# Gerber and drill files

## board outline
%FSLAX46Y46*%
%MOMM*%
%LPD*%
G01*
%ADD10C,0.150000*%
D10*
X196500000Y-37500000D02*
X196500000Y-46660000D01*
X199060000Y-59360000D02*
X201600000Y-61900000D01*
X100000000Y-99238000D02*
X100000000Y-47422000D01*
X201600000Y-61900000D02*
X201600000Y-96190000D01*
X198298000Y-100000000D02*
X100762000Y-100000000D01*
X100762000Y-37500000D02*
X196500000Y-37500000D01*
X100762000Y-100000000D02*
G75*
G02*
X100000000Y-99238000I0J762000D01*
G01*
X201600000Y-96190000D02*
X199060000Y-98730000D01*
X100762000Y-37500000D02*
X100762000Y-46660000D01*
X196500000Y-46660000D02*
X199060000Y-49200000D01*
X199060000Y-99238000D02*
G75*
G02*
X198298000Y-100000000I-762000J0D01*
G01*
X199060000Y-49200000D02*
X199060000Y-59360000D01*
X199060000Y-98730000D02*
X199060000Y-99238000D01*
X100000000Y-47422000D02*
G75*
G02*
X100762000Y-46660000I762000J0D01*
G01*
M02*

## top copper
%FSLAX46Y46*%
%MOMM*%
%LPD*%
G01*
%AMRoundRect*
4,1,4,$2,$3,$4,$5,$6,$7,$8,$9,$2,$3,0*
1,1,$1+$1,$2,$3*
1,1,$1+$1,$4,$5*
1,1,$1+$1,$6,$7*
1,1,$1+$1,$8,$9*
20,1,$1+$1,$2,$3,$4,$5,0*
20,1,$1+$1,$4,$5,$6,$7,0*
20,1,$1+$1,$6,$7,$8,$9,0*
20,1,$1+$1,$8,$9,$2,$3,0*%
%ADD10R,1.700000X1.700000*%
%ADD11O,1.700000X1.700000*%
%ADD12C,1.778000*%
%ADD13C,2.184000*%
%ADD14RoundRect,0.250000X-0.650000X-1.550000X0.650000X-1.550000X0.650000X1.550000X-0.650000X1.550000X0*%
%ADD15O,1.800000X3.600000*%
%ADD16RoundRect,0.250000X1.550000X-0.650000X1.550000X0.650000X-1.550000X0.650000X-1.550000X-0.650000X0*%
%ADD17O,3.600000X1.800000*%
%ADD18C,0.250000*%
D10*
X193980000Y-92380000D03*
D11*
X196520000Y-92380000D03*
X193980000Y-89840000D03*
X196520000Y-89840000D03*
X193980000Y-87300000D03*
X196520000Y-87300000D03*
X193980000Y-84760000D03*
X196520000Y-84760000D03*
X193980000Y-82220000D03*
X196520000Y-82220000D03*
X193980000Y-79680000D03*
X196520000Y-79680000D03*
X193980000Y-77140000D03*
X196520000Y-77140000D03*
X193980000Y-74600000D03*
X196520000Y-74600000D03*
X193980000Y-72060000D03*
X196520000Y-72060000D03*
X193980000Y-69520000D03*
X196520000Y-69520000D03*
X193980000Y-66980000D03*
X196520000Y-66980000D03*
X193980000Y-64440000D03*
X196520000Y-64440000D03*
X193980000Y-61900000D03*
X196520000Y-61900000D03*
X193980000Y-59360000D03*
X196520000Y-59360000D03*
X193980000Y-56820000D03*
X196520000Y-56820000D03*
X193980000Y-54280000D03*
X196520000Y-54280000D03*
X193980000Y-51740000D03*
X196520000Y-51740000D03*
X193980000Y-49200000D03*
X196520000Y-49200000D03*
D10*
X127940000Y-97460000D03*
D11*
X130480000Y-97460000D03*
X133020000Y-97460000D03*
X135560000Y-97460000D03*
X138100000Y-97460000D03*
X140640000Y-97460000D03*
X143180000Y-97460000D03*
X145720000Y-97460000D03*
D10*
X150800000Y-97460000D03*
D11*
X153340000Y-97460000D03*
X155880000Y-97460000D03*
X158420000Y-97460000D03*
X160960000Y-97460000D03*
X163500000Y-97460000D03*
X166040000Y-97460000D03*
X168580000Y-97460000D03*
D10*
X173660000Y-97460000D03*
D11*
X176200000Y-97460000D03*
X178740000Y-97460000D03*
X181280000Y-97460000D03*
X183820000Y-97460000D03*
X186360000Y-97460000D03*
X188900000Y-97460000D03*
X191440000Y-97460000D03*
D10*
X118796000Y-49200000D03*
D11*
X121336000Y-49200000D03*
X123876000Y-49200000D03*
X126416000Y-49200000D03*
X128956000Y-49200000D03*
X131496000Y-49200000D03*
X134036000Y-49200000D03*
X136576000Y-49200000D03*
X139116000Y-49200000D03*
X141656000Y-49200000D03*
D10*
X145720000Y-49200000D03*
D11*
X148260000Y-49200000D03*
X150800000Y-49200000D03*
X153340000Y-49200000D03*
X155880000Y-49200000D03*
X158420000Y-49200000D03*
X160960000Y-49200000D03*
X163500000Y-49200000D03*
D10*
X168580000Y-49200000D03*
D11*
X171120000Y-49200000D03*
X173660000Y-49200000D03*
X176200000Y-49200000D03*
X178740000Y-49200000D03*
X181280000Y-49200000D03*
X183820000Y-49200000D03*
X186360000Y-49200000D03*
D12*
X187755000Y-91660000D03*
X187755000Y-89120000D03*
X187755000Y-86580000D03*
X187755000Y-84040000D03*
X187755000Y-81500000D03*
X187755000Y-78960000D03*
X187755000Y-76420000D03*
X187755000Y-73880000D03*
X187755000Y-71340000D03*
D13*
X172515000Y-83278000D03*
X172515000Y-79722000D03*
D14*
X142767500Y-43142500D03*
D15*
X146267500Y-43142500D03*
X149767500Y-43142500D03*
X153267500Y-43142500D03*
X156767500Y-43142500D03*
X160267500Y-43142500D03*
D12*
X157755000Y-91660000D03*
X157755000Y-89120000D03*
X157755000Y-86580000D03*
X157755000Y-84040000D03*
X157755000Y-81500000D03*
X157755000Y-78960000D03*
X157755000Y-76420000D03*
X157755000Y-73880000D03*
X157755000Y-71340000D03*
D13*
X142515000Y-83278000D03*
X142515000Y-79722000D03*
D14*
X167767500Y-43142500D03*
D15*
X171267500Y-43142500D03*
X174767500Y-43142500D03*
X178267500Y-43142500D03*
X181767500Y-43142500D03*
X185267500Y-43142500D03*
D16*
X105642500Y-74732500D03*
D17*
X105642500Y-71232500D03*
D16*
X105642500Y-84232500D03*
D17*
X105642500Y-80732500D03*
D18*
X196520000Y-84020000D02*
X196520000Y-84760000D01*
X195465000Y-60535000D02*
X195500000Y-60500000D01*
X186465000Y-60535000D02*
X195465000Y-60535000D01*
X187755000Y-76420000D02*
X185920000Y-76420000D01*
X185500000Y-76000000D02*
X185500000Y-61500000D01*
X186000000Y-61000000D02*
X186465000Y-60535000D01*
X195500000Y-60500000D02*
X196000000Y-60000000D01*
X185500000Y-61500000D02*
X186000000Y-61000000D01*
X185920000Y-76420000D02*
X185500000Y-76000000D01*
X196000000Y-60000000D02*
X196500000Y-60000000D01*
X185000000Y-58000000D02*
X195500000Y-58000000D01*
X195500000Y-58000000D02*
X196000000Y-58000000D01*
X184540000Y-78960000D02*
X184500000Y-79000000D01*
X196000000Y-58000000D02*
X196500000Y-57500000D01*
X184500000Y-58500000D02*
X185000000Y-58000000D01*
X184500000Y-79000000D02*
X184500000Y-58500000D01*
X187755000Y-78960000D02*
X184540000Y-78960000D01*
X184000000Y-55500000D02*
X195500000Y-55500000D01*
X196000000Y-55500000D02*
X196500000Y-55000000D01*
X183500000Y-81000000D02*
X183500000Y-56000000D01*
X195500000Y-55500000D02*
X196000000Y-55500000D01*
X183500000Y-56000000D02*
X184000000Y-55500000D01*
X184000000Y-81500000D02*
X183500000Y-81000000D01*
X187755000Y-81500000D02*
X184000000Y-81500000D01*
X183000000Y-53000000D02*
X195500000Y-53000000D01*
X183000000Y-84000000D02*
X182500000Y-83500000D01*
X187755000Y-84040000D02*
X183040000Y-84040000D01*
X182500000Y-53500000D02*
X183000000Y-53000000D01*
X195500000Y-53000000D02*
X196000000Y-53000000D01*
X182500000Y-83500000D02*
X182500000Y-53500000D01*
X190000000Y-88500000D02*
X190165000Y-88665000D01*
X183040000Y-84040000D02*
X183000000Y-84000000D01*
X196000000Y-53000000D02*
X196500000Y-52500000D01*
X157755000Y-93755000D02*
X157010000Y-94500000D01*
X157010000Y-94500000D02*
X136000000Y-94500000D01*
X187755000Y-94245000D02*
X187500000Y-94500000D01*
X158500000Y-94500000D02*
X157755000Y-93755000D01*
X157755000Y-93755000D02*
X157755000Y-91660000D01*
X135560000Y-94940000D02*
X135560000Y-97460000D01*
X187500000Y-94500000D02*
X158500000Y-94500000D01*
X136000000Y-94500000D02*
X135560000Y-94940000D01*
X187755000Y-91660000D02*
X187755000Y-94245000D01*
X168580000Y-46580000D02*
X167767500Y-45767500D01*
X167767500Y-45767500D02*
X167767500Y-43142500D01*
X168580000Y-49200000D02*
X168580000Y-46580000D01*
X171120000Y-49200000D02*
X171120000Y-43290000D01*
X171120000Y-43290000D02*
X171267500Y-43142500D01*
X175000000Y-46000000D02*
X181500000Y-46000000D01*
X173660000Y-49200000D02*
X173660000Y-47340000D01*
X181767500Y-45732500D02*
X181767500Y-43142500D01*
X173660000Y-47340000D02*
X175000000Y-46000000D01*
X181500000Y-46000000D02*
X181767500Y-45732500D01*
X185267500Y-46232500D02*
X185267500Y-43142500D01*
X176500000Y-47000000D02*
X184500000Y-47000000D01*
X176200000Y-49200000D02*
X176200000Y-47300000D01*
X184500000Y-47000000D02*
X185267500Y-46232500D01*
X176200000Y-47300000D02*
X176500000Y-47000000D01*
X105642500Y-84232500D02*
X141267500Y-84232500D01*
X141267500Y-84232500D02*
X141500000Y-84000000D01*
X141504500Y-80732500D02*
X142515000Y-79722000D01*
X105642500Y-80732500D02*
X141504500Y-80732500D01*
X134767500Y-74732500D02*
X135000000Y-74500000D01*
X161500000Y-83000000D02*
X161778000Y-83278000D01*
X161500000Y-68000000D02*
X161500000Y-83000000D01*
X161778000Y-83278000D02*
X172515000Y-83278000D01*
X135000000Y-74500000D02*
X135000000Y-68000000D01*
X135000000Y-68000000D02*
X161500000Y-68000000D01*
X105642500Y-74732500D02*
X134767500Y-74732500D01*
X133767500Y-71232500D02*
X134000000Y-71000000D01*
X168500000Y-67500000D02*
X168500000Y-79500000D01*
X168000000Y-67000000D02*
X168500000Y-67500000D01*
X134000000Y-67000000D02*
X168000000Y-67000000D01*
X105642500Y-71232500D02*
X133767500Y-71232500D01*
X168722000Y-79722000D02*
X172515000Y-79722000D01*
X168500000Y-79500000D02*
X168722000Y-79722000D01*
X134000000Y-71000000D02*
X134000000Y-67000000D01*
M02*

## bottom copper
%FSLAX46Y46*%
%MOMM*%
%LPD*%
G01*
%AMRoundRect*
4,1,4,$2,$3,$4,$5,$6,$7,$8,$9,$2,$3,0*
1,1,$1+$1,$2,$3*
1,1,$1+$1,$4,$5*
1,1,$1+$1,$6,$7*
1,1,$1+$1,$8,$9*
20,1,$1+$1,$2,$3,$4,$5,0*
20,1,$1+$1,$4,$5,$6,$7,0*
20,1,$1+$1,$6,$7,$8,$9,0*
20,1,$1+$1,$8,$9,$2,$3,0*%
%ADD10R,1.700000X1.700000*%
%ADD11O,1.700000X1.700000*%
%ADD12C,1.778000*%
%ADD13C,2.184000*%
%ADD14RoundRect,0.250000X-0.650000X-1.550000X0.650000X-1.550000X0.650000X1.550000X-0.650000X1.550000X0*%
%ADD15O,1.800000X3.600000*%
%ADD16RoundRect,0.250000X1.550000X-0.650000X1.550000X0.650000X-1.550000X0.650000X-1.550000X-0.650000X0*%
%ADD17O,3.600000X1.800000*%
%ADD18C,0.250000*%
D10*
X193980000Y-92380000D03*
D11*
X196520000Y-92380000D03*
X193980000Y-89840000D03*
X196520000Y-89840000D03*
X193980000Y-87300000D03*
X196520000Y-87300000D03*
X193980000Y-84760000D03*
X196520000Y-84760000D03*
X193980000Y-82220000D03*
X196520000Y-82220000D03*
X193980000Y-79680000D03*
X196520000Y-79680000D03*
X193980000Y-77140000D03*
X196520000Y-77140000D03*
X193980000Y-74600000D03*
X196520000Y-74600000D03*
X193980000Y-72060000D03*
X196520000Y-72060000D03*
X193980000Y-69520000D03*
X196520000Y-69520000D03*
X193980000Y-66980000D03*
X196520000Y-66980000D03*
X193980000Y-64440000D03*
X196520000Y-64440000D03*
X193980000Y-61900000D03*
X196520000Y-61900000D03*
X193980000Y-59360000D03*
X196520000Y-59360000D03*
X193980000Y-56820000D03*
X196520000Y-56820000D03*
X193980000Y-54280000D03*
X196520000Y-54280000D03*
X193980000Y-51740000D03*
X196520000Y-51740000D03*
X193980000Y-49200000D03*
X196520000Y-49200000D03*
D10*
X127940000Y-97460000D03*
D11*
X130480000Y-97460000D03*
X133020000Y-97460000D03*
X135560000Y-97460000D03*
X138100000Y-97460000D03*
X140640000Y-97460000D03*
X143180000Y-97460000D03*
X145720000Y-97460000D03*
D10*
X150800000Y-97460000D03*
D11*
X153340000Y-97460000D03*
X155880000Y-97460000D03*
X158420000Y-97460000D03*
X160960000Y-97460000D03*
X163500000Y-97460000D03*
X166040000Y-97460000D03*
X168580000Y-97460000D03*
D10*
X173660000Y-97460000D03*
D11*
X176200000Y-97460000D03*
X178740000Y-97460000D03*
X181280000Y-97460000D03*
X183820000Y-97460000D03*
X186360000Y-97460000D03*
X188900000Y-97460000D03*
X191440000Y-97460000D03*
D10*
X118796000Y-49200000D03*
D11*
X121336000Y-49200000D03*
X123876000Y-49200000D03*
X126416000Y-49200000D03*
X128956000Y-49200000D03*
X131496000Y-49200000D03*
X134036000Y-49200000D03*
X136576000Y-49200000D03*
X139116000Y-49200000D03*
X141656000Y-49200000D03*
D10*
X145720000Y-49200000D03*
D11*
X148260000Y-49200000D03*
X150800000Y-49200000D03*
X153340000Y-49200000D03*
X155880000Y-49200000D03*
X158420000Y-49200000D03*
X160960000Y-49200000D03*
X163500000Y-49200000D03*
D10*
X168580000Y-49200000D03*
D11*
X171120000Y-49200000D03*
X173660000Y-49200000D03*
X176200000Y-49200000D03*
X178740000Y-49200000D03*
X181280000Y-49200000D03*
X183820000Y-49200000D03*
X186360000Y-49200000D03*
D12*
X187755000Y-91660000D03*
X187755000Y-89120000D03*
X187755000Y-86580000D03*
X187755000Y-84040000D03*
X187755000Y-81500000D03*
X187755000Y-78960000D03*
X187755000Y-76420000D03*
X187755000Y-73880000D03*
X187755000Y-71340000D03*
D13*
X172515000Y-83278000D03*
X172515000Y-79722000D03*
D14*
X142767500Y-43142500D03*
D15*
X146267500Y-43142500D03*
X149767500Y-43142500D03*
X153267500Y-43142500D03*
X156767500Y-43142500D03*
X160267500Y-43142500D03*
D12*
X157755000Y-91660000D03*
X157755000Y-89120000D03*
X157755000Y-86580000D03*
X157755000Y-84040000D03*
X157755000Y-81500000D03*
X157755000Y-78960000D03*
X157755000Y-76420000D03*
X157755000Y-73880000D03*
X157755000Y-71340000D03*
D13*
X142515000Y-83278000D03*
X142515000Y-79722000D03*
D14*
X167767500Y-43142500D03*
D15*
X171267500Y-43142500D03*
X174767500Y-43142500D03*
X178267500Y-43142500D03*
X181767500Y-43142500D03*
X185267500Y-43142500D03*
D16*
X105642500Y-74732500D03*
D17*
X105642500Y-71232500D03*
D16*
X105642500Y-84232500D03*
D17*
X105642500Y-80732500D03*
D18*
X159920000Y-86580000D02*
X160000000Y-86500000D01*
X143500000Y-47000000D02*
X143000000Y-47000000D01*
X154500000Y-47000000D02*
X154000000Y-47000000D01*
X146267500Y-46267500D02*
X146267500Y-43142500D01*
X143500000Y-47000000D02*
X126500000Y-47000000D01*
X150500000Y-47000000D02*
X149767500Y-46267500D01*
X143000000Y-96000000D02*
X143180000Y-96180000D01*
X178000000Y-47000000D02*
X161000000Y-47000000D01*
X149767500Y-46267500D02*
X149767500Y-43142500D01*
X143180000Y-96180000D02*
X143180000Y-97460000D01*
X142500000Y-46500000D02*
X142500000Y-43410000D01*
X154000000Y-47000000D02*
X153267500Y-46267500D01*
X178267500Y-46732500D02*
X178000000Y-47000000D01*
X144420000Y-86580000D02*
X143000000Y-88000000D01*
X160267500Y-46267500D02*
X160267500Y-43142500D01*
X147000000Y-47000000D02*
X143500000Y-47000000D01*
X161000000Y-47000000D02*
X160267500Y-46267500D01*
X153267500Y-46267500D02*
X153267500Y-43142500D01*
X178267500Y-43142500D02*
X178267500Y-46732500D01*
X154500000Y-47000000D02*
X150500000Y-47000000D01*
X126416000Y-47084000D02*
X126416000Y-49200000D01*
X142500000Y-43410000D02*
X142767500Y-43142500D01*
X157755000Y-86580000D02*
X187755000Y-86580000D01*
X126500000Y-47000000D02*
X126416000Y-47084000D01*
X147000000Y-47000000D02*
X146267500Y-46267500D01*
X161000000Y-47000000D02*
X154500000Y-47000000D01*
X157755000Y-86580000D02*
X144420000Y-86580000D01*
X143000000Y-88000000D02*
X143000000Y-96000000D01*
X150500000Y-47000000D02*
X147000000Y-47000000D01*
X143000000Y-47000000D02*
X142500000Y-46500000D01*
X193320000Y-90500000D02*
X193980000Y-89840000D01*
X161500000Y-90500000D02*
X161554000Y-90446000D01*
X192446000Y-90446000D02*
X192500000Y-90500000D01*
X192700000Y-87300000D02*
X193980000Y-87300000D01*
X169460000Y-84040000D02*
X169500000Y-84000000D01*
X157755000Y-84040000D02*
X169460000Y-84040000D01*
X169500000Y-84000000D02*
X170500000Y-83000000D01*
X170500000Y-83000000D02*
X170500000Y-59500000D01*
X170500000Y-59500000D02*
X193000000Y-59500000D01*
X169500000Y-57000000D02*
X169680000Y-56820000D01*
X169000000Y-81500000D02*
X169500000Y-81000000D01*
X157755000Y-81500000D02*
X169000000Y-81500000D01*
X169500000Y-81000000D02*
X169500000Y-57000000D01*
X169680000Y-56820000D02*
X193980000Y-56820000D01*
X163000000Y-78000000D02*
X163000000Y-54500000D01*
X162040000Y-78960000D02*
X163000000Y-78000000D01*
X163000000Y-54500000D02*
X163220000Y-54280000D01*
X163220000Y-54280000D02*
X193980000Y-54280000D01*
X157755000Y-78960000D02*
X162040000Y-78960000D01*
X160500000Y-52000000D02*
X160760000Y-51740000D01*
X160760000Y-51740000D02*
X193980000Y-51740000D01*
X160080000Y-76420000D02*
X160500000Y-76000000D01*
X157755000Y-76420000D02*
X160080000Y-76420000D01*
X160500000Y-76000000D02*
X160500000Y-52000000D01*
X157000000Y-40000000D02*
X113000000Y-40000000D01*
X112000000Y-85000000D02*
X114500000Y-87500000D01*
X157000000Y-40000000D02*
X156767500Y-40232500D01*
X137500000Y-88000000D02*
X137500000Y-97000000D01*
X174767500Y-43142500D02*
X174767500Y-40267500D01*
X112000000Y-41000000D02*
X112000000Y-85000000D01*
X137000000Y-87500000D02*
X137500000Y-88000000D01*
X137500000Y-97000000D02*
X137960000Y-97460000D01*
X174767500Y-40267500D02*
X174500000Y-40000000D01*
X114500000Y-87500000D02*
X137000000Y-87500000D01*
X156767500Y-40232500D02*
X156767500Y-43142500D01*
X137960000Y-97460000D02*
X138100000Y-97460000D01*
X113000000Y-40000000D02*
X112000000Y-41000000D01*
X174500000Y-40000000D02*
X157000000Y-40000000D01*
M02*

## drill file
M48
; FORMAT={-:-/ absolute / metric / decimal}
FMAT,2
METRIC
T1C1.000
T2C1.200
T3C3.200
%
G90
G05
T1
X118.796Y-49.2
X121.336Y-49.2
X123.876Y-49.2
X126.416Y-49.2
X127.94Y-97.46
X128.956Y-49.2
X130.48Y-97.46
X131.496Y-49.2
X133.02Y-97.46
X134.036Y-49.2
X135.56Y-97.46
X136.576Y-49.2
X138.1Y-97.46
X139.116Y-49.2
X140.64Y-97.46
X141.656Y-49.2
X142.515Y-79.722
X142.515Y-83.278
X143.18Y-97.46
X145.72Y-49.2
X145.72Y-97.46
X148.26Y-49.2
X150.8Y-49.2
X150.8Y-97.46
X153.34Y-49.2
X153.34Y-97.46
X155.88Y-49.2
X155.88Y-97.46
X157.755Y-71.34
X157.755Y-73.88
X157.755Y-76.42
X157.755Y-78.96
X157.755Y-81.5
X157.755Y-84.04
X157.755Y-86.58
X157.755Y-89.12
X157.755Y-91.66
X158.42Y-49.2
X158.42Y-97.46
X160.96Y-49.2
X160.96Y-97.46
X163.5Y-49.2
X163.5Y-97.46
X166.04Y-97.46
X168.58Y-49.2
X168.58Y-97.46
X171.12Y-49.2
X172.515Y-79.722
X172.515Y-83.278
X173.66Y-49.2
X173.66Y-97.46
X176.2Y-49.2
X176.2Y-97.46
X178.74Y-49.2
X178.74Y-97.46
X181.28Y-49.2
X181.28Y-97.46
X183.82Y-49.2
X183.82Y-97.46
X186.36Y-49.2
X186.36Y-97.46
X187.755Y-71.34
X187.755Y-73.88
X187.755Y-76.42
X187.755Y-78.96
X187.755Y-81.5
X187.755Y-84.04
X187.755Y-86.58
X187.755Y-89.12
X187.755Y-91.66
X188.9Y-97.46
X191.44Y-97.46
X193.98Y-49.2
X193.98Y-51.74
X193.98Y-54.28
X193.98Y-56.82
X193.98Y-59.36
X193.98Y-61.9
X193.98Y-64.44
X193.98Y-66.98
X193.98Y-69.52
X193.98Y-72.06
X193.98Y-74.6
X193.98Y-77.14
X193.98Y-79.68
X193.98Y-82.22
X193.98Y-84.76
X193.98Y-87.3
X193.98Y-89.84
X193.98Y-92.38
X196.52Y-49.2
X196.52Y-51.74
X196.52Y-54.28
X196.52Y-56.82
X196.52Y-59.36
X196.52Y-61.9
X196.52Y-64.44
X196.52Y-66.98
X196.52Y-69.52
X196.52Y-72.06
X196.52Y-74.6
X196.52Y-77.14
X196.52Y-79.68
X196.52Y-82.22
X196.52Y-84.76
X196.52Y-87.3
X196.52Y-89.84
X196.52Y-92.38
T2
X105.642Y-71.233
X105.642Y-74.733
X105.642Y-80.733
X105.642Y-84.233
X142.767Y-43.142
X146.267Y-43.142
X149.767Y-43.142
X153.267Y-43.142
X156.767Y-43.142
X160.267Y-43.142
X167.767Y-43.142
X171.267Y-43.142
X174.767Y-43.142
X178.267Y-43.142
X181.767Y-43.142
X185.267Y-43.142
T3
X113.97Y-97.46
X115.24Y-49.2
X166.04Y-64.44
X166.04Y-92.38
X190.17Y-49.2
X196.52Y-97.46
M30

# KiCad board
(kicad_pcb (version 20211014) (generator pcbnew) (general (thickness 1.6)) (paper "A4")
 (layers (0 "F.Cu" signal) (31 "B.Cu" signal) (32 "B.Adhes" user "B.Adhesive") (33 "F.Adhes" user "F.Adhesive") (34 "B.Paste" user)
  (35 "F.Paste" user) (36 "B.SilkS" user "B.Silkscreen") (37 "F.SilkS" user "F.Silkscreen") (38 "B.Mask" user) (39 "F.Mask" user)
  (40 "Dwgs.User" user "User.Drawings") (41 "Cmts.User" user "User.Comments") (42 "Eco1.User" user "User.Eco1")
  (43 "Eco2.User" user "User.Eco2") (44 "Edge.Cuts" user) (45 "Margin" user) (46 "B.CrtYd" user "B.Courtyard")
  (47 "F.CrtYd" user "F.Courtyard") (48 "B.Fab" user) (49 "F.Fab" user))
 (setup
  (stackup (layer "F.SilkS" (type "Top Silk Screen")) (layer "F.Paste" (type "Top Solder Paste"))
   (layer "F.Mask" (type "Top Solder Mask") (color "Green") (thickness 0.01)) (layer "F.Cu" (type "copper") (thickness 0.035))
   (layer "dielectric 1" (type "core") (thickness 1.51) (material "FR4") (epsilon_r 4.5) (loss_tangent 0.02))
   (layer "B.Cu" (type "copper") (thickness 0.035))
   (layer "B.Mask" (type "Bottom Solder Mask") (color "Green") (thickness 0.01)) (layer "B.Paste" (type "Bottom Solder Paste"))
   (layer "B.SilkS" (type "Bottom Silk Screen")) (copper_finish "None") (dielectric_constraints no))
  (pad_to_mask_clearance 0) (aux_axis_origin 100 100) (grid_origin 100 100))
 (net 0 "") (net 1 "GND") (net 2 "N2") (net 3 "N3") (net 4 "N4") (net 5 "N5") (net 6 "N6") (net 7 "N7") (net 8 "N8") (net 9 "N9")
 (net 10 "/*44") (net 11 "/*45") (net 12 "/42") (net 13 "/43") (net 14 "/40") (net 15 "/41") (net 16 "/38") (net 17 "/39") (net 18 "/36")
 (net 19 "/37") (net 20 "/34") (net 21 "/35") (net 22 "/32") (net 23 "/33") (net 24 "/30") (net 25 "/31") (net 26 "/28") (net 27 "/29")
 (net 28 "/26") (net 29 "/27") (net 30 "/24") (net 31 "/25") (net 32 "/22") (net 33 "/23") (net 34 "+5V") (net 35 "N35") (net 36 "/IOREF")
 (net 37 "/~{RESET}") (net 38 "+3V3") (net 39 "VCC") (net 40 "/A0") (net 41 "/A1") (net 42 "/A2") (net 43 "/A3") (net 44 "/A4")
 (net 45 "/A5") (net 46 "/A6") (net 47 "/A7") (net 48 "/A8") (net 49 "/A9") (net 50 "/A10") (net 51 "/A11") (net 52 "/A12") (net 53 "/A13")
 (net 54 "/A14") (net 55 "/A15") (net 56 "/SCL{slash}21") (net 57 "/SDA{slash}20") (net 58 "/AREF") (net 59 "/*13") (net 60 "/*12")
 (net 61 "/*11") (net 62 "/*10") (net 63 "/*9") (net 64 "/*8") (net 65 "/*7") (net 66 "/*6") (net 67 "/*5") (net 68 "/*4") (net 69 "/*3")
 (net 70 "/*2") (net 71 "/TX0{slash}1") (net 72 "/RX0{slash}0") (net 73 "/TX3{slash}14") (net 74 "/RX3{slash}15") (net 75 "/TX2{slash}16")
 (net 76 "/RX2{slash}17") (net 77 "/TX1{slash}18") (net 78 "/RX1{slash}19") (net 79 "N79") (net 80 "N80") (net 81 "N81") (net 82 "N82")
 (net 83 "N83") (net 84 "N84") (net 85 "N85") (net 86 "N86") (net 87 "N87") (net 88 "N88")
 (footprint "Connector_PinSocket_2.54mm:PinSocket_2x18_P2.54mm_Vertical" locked (layer "F.Cu") (at 193.98 92.38 180)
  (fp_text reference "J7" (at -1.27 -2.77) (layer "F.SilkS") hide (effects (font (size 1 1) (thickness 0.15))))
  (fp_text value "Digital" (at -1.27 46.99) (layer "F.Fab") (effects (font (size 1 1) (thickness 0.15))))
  (pad "1" thru_hole rect locked (at 0 0 180) (size 1.7 1.7) (drill 1) (layers *.Cu *.Mask) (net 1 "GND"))
  (pad "2" thru_hole oval locked (at -2.54 0 180) (size 1.7 1.7) (drill 1) (layers *.Cu *.Mask) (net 1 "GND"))
  (pad "3" thru_hole oval locked (at 0 2.54 180) (size 1.7 1.7) (drill 1) (layers *.Cu *.Mask) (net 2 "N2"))
  (pad "4" thru_hole oval locked (at -2.54 2.54 180) (size 1.7 1.7) (drill 1) (layers *.Cu *.Mask) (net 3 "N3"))
  (pad "5" thru_hole oval locked (at 0 5.08 180) (size 1.7 1.7) (drill 1) (layers *.Cu *.Mask) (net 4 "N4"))
  (pad "6" thru_hole oval locked (at -2.54 5.08 180) (size 1.7 1.7) (drill 1) (layers *.Cu *.Mask) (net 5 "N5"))
  (pad "7" thru_hole oval locked (at 0 7.62 180) (size 1.7 1.7) (drill 1) (layers *.Cu *.Mask) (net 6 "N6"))
  (pad "8" thru_hole oval locked (at -2.54 7.62 180) (size 1.7 1.7) (drill 1) (layers *.Cu *.Mask) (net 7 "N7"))
  (pad "9" thru_hole oval locked (at 0 10.16 180) (size 1.7 1.7) (drill 1) (layers *.Cu *.Mask) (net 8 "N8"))
  (pad "10" thru_hole oval locked (at -2.54 10.16 180) (size 1.7 1.7) (drill 1) (layers *.Cu *.Mask) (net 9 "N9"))
  (pad "11" thru_hole oval locked (at 0 12.7 180) (size 1.7 1.7) (drill 1) (layers *.Cu *.Mask) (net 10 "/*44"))
  (pad "12" thru_hole oval locked (at -2.54 12.7 180) (size 1.7 1.7) (drill 1) (layers *.Cu *.Mask) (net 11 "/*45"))
  (pad "13" thru_hole oval locked (at 0 15.24 180) (size 1.7 1.7) (drill 1) (layers *.Cu *.Mask) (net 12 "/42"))
  (pad "14" thru_hole oval locked (at -2.54 15.24 180) (size 1.7 1.7) (drill 1) (layers *.Cu *.Mask) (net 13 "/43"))
  (pad "15" thru_hole oval locked (at 0 17.78 180) (size 1.7 1.7) (drill 1) (layers *.Cu *.Mask) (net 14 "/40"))
  (pad "16" thru_hole oval locked (at -2.54 17.78 180) (size 1.7 1.7) (drill 1) (layers *.Cu *.Mask) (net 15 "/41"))
  (pad "17" thru_hole oval locked (at 0 20.32 180) (size 1.7 1.7) (drill 1) (layers *.Cu *.Mask) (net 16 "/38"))
  (pad "18" thru_hole oval locked (at -2.54 20.32 180) (size 1.7 1.7) (drill 1) (layers *.Cu *.Mask) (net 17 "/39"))
  (pad "19" thru_hole oval locked (at 0 22.86 180) (size 1.7 1.7) (drill 1) (layers *.Cu *.Mask) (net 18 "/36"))
  (pad "20" thru_hole oval locked (at -2.54 22.86 180) (size 1.7 1.7) (drill 1) (layers *.Cu *.Mask) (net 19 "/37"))
  (pad "21" thru_hole oval locked (at 0 25.4 180) (size 1.7 1.7) (drill 1) (layers *.Cu *.Mask) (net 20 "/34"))
  (pad "22" thru_hole oval locked (at -2.54 25.4 180) (size 1.7 1.7) (drill 1) (layers *.Cu *.Mask) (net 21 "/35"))
  (pad "23" thru_hole oval locked (at 0 27.94 180) (size 1.7 1.7) (drill 1) (layers *.Cu *.Mask) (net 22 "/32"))
  (pad "24" thru_hole oval locked (at -2.54 27.94 180) (size 1.7 1.7) (drill 1) (layers *.Cu *.Mask) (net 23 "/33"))
  (pad "25" thru_hole oval locked (at 0 30.48 180) (size 1.7 1.7) (drill 1) (layers *.Cu *.Mask) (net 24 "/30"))
  (pad "26" thru_hole oval locked (at -2.54 30.48 180) (size 1.7 1.7) (drill 1) (layers *.Cu *.Mask) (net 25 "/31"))
  (pad "27" thru_hole oval locked (at 0 33.02 180) (size 1.7 1.7) (drill 1) (layers *.Cu *.Mask) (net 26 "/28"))
  (pad "28" thru_hole oval locked (at -2.54 33.02 180) (size 1.7 1.7) (drill 1) (layers *.Cu *.Mask) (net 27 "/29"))
  (pad "29" thru_hole oval locked (at 0 35.56 180) (size 1.7 1.7) (drill 1) (layers *.Cu *.Mask) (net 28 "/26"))
  (pad "30" thru_hole oval locked (at -2.54 35.56 180) (size 1.7 1.7) (drill 1) (layers *.Cu *.Mask) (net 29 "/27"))
  (pad "31" thru_hole oval locked (at 0 38.1 180) (size 1.7 1.7) (drill 1) (layers *.Cu *.Mask) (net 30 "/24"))
  (pad "32" thru_hole oval locked (at -2.54 38.1 180) (size 1.7 1.7) (drill 1) (layers *.Cu *.Mask) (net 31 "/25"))
  (pad "33" thru_hole oval locked (at 0 40.64 180) (size 1.7 1.7) (drill 1) (layers *.Cu *.Mask) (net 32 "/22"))
  (pad "34" thru_hole oval locked (at -2.54 40.64 180) (size 1.7 1.7) (drill 1) (layers *.Cu *.Mask) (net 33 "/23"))
  (pad "35" thru_hole oval locked (at 0 43.18 180) (size 1.7 1.7) (drill 1) (layers *.Cu *.Mask) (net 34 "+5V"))
  (pad "36" thru_hole oval locked (at -2.54 43.18 180) (size 1.7 1.7) (drill 1) (layers *.Cu *.Mask) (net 34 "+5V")))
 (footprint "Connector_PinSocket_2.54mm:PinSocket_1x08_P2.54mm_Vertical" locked (layer "F.Cu") (at 127.94 97.46 90)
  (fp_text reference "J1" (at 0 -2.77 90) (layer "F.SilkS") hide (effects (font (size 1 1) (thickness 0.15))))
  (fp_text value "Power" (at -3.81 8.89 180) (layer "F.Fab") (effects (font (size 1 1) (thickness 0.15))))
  (pad "1" thru_hole rect locked (at 0 0 90) (size 1.7 1.7) (drill 1) (layers *.Cu *.Mask) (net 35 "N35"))
  (pad "2" thru_hole oval locked (at 0 2.54 90) (size 1.7 1.7) (drill 1) (layers *.Cu *.Mask) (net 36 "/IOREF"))
  (pad "3" thru_hole oval locked (at 0 5.08 90) (size 1.7 1.7) (drill 1) (layers *.Cu *.Mask) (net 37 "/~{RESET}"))
  (pad "4" thru_hole oval locked (at 0 7.62 90) (size 1.7 1.7) (drill 1) (layers *.Cu *.Mask) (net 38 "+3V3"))
  (pad "5" thru_hole oval locked (at 0 10.16 90) (size 1.7 1.7) (drill 1) (layers *.Cu *.Mask) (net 34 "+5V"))
  (pad "6" thru_hole oval locked (at 0 12.7 90) (size 1.7 1.7) (drill 1) (layers *.Cu *.Mask) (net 1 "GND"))
  (pad "7" thru_hole oval locked (at 0 15.24 90) (size 1.7 1.7) (drill 1) (layers *.Cu *.Mask) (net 1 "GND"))
  (pad "8" thru_hole oval locked (at 0 17.78 90) (size 1.7 1.7) (drill 1) (layers *.Cu *.Mask) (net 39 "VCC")))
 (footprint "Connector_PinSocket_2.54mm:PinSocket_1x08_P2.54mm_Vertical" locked (layer "F.Cu") (at 150.8 97.46 90)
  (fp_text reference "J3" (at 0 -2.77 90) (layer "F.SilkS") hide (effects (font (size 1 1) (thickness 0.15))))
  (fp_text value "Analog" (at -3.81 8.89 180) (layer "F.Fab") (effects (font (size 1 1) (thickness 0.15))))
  (pad "1" thru_hole rect locked (at 0 0 90) (size 1.7 1.7) (drill 1) (layers *.Cu *.Mask) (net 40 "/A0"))
  (pad "2" thru_hole oval locked (at 0 2.54 90) (size 1.7 1.7) (drill 1) (layers *.Cu *.Mask) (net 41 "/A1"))
  (pad "3" thru_hole oval locked (at 0 5.08 90) (size 1.7 1.7) (drill 1) (layers *.Cu *.Mask) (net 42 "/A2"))
  (pad "4" thru_hole oval locked (at 0 7.62 90) (size 1.7 1.7) (drill 1) (layers *.Cu *.Mask) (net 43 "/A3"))
  (pad "5" thru_hole oval locked (at 0 10.16 90) (size 1.7 1.7) (drill 1) (layers *.Cu *.Mask) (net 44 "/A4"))
  (pad "6" thru_hole oval locked (at 0 12.7 90) (size 1.7 1.7) (drill 1) (layers *.Cu *.Mask) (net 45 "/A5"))
  (pad "7" thru_hole oval locked (at 0 15.24 90) (size 1.7 1.7) (drill 1) (layers *.Cu *.Mask) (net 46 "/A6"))
  (pad "8" thru_hole oval locked (at 0 17.78 90) (size 1.7 1.7) (drill 1) (layers *.Cu *.Mask) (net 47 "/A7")))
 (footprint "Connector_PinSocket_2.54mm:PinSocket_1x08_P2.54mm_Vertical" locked (layer "F.Cu") (at 173.66 97.46 90)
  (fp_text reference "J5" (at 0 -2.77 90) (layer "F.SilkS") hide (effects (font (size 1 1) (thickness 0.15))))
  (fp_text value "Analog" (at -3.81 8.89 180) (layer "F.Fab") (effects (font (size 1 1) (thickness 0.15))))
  (pad "1" thru_hole rect locked (at 0 0 90) (size 1.7 1.7) (drill 1) (layers *.Cu *.Mask) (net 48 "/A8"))
  (pad "2" thru_hole oval locked (at 0 2.54 90) (size 1.7 1.7) (drill 1) (layers *.Cu *.Mask) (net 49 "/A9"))
  (pad "3" thru_hole oval locked (at 0 5.08 90) (size 1.7 1.7) (drill 1) (layers *.Cu *.Mask) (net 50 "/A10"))
  (pad "4" thru_hole oval locked (at 0 7.62 90) (size 1.7 1.7) (drill 1) (layers *.Cu *.Mask) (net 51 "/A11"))
  (pad "5" thru_hole oval locked (at 0 10.16 90) (size 1.7 1.7) (drill 1) (layers *.Cu *.Mask) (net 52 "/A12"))
  (pad "6" thru_hole oval locked (at 0 12.7 90) (size 1.7 1.7) (drill 1) (layers *.Cu *.Mask) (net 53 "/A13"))
  (pad "7" thru_hole oval locked (at 0 15.24 90) (size 1.7 1.7) (drill 1) (layers *.Cu *.Mask) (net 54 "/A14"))
  (pad "8" thru_hole oval locked (at 0 17.78 90) (size 1.7 1.7) (drill 1) (layers *.Cu *.Mask) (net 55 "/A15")))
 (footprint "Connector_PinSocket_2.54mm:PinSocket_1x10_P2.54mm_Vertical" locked (layer "F.Cu") (at 118.796 49.2 90)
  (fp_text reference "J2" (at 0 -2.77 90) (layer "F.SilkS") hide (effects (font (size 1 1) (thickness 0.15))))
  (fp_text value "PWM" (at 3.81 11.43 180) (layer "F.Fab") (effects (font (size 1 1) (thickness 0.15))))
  (pad "1" thru_hole rect locked (at 0 0 90) (size 1.7 1.7) (drill 1) (layers *.Cu *.Mask) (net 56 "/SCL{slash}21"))
  (pad "2" thru_hole oval locked (at 0 2.54 90) (size 1.7 1.7) (drill 1) (layers *.Cu *.Mask) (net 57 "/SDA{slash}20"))
  (pad "3" thru_hole oval locked (at 0 5.08 90) (size 1.7 1.7) (drill 1) (layers *.Cu *.Mask) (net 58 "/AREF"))
  (pad "4" thru_hole oval locked (at 0 7.62 90) (size 1.7 1.7) (drill 1) (layers *.Cu *.Mask) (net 1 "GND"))
  (pad "5" thru_hole oval locked (at 0 10.16 90) (size 1.7 1.7) (drill 1) (layers *.Cu *.Mask) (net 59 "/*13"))
  (pad "6" thru_hole oval locked (at 0 12.7 90) (size 1.7 1.7) (drill 1) (layers *.Cu *.Mask) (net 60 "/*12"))
  (pad "7" thru_hole oval locked (at 0 15.24 90) (size 1.7 1.7) (drill 1) (layers *.Cu *.Mask) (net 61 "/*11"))
  (pad "8" thru_hole oval locked (at 0 17.78 90) (size 1.7 1.7) (drill 1) (layers *.Cu *.Mask) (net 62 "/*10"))
  (pad "9" thru_hole oval locked (at 0 20.32 90) (size 1.7 1.7) (drill 1) (layers *.Cu *.Mask) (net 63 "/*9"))
  (pad "10" thru_hole oval locked (at 0 22.86 90) (size 1.7 1.7) (drill 1) (layers *.Cu *.Mask) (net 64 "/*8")))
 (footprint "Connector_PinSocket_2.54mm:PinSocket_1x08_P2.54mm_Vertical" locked (layer "F.Cu") (at 145.72 49.2 90)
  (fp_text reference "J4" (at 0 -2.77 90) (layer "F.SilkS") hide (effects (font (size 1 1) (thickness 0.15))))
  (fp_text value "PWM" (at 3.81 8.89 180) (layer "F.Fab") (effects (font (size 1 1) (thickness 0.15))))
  (pad "1" thru_hole rect locked (at 0 0 90) (size 1.7 1.7) (drill 1) (layers *.Cu *.Mask) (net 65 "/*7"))
  (pad "2" thru_hole oval locked (at 0 2.54 90) (size 1.7 1.7) (drill 1) (layers *.Cu *.Mask) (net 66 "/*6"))
  (pad "3" thru_hole oval locked (at 0 5.08 90) (size 1.7 1.7) (drill 1) (layers *.Cu *.Mask) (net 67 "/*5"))
  (pad "4" thru_hole oval locked (at 0 7.62 90) (size 1.7 1.7) (drill 1) (layers *.Cu *.Mask) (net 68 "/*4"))
  (pad "5" thru_hole oval locked (at 0 10.16 90) (size 1.7 1.7) (drill 1) (layers *.Cu *.Mask) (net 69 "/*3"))
  (pad "6" thru_hole oval locked (at 0 12.7 90) (size 1.7 1.7) (drill 1) (layers *.Cu *.Mask) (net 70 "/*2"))
  (pad "7" thru_hole oval locked (at 0 15.24 90) (size 1.7 1.7) (drill 1) (layers *.Cu *.Mask) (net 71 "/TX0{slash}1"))
  (pad "8" thru_hole oval locked (at 0 17.78 90) (size 1.7 1.7) (drill 1) (layers *.Cu *.Mask) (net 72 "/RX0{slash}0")))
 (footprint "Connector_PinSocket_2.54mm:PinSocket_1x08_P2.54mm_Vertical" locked (layer "F.Cu") (at 168.58 49.2 90)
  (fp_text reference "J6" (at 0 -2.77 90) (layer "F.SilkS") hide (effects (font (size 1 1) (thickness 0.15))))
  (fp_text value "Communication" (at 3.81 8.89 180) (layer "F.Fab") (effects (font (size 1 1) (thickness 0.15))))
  (pad "1" thru_hole rect locked (at 0 0 90) (size 1.7 1.7) (drill 1) (layers *.Cu *.Mask) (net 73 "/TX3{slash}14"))
  (pad "2" thru_hole oval locked (at 0 2.54 90) (size 1.7 1.7) (drill 1) (layers *.Cu *.Mask) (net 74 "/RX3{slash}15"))
  (pad "3" thru_hole oval locked (at 0 5.08 90) (size 1.7 1.7) (drill 1) (layers *.Cu *.Mask) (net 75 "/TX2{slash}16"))
  (pad "4" thru_hole oval locked (at 0 7.62 90) (size 1.7 1.7) (drill 1) (layers *.Cu *.Mask) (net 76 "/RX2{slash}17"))
  (pad "5" thru_hole oval locked (at 0 10.16 90) (size 1.7 1.7) (drill 1) (layers *.Cu *.Mask) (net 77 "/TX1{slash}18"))
  (pad "6" thru_hole oval locked (at 0 12.7 90) (size 1.7 1.7) (drill 1) (layers *.Cu *.Mask) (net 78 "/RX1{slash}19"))
  (pad "7" thru_hole oval locked (at 0 15.24 90) (size 1.7 1.7) (drill 1) (layers *.Cu *.Mask) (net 57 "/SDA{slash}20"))
  (pad "8" thru_hole oval locked (at 0 17.78 90) (size 1.7 1.7) (drill 1) (layers *.Cu *.Mask) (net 56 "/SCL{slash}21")))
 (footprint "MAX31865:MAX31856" (layer "F.Cu") (at 179.5 81.5 90)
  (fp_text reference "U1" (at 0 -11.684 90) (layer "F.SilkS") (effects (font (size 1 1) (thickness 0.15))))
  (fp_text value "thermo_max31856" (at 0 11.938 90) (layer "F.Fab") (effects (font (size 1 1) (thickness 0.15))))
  (pad "1" thru_hole circle (at -10.16 8.255 90) (size 1.778 1.778) (drill 1) (layers *.Cu *.Mask) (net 38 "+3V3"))
  (pad "2" thru_hole circle (at -7.62 8.255 90) (size 1.778 1.778) (drill 1) (layers *.Cu *.Mask) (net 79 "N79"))
  (pad "3" thru_hole circle (at -5.08 8.255 90) (size 1.778 1.778) (drill 1) (layers *.Cu *.Mask) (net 1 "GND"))
  (pad "4" thru_hole circle (at -2.54 8.255 90) (size 1.778 1.778) (drill 1) (layers *.Cu *.Mask) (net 33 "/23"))
  (pad "5" thru_hole circle (at 0 8.255 90) (size 1.778 1.778) (drill 1) (layers *.Cu *.Mask) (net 31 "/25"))
  (pad "6" thru_hole circle (at 2.54 8.255 90) (size 1.778 1.778) (drill 1) (layers *.Cu *.Mask) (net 29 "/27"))
  (pad "7" thru_hole circle (at 5.08 8.255 90) (size 1.778 1.778) (drill 1) (layers *.Cu *.Mask) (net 27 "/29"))
  (pad "8" thru_hole circle (at 7.62 8.255 90) (size 1.778 1.778) (drill 1) (layers *.Cu *.Mask) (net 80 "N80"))
  (pad "9" thru_hole circle (at 10.16 8.255 90) (size 1.778 1.778) (drill 1) (layers *.Cu *.Mask) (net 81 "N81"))
  (pad "10" thru_hole circle (at -1.778 -6.985 90) (size 2.184 2.184) (drill 1) (layers *.Cu *.Mask) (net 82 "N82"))
  (pad "11" thru_hole circle (at 1.778 -6.985 90) (size 2.184 2.184) (drill 1) (layers *.Cu *.Mask) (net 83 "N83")))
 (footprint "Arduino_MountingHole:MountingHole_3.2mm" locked (layer "F.Cu") (at 196.52 97.46)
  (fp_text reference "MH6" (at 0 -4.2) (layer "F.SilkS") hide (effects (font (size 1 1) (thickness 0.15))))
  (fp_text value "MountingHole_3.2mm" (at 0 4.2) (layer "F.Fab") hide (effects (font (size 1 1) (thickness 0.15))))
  (pad "" np_thru_hole circle locked (at 0 0) (size 3.2 3.2) (drill 3.2) (layers *.Cu *.Mask)))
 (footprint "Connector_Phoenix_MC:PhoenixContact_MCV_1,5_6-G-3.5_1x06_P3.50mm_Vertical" (layer "F.Cu") (at 142.7675 43.1425)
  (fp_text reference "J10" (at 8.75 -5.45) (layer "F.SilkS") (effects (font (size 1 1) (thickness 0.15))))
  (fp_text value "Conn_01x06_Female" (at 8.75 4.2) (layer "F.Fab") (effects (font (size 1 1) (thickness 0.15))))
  (pad "1" thru_hole roundrect (at 0 0) (size 1.8 3.6) (drill 1.2) (layers *.Cu *.Mask) (roundrect_rratio 0.138889) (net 1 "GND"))
  (pad "2" thru_hole oval (at 3.5 0) (size 1.8 3.6) (drill 1.2) (layers *.Cu *.Mask) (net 1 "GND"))
  (pad "3" thru_hole oval (at 7 0) (size 1.8 3.6) (drill 1.2) (layers *.Cu *.Mask) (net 1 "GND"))
  (pad "4" thru_hole oval (at 10.5 0) (size 1.8 3.6) (drill 1.2) (layers *.Cu *.Mask) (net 1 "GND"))
  (pad "5" thru_hole oval (at 14 0) (size 1.8 3.6) (drill 1.2) (layers *.Cu *.Mask) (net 34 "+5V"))
  (pad "6" thru_hole oval (at 17.5 0) (size 1.8 3.6) (drill 1.2) (layers *.Cu *.Mask) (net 1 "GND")))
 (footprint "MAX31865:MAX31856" (layer "F.Cu") (at 149.5 81.5 90)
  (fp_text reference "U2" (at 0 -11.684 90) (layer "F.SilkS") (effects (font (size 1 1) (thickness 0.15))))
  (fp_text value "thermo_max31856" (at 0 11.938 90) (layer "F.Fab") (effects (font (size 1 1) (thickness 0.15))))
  (pad "1" thru_hole circle (at -10.16 8.255 90) (size 1.778 1.778) (drill 1) (layers *.Cu *.Mask) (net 38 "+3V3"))
  (pad "2" thru_hole circle (at -7.62 8.255 90) (size 1.778 1.778) (drill 1) (layers *.Cu *.Mask) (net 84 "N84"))
  (pad "3" thru_hole circle (at -5.08 8.255 90) (size 1.778 1.778) (drill 1) (layers *.Cu *.Mask) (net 1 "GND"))
  (pad "4" thru_hole circle (at -2.54 8.255 90) (size 1.778 1.778) (drill 1) (layers *.Cu *.Mask) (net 26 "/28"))
  (pad "5" thru_hole circle (at 0 8.255 90) (size 1.778 1.778) (drill 1) (layers *.Cu *.Mask) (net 28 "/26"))
  (pad "6" thru_hole circle (at 2.54 8.255 90) (size 1.778 1.778) (drill 1) (layers *.Cu *.Mask) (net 30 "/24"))
  (pad "7" thru_hole circle (at 5.08 8.255 90) (size 1.778 1.778) (drill 1) (layers *.Cu *.Mask) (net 32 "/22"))
  (pad "8" thru_hole circle (at 7.62 8.255 90) (size 1.778 1.778) (drill 1) (layers *.Cu *.Mask) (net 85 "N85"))
  (pad "9" thru_hole circle (at 10.16 8.255 90) (size 1.778 1.778) (drill 1) (layers *.Cu *.Mask) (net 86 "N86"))
  (pad "10" thru_hole circle (at -1.778 -6.985 90) (size 2.184 2.184) (drill 1) (layers *.Cu *.Mask) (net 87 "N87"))
  (pad "11" thru_hole circle (at 1.778 -6.985 90) (size 2.184 2.184) (drill 1) (layers *.Cu *.Mask) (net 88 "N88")))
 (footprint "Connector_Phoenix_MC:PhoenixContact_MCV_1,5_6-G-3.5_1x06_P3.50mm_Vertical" (layer "F.Cu") (at 167.7675 43.1425)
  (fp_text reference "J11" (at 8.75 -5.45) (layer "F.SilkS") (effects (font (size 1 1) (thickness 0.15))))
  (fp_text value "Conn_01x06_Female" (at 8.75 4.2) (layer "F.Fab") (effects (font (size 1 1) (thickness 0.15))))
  (pad "1" thru_hole roundrect (at 0 0) (size 1.8 3.6) (drill 1.2) (layers *.Cu *.Mask) (roundrect_rratio 0.138889) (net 73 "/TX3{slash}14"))
  (pad "2" thru_hole oval (at 3.5 0) (size 1.8 3.6) (drill 1.2) (layers *.Cu *.Mask) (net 74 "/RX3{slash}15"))
  (pad "3" thru_hole oval (at 7 0) (size 1.8 3.6) (drill 1.2) (layers *.Cu *.Mask) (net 34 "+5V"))
  (pad "4" thru_hole oval (at 10.5 0) (size 1.8 3.6) (drill 1.2) (layers *.Cu *.Mask) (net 1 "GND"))
  (pad "5" thru_hole oval (at 14 0) (size 1.8 3.6) (drill 1.2) (layers *.Cu *.Mask) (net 75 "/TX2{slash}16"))
  (pad "6" thru_hole oval (at 17.5 0) (size 1.8 3.6) (drill 1.2) (layers *.Cu *.Mask) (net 76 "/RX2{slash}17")))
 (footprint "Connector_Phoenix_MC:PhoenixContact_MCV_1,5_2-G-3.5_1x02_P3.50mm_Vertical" (layer "F.Cu") (at 105.6425 74.7325 90)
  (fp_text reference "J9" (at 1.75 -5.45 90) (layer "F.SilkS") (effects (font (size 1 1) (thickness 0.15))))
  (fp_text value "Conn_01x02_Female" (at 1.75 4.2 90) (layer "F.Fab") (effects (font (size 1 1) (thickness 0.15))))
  (pad "1" thru_hole roundrect (at 0 0 90) (size 1.8 3.6) (drill 1.2) (layers *.Cu *.Mask) (roundrect_rratio 0.138889) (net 82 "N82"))
  (pad "2" thru_hole oval (at 3.5 0 90) (size 1.8 3.6) (drill 1.2) (layers *.Cu *.Mask) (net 83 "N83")))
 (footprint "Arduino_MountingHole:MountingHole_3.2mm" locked (layer "F.Cu") (at 115.24 49.2)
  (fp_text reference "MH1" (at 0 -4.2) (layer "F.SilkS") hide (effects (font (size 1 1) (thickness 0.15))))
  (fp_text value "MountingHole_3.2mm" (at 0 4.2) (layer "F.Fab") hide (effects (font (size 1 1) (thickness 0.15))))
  (pad "" np_thru_hole circle locked (at 0 0) (size 3.2 3.2) (drill 3.2) (layers *.Cu *.Mask)))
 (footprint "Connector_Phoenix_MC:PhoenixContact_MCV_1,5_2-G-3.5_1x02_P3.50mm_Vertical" (layer "F.Cu") (at 105.6425 84.2325 90)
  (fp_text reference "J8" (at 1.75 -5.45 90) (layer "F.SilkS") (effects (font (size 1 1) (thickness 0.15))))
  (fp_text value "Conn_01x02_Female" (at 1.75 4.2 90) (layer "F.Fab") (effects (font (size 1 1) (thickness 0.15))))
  (pad "1" thru_hole roundrect (at 0 0 90) (size 1.8 3.6) (drill 1.2) (layers *.Cu *.Mask) (roundrect_rratio 0.138889) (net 87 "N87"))
  (pad "2" thru_hole oval (at 3.5 0 90) (size 1.8 3.6) (drill 1.2) (layers *.Cu *.Mask) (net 88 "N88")))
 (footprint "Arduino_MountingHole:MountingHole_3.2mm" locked (layer "F.Cu") (at 113.97 97.46)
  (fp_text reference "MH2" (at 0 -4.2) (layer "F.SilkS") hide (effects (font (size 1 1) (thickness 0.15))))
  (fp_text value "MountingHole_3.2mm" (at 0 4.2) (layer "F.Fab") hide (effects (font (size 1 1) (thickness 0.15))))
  (pad "" np_thru_hole circle locked (at 0 0) (size 3.2 3.2) (drill 3.2) (layers *.Cu *.Mask)))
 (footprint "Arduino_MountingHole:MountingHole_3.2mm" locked (layer "F.Cu") (at 166.04 64.44)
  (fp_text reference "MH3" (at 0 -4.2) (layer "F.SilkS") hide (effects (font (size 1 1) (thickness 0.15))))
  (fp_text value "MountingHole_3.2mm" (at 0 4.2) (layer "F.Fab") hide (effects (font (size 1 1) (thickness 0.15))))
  (pad "" np_thru_hole circle locked (at 0 0) (size 3.2 3.2) (drill 3.2) (layers *.Cu *.Mask)))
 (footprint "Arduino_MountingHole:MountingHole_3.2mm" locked (layer "F.Cu") (at 166.04 92.38)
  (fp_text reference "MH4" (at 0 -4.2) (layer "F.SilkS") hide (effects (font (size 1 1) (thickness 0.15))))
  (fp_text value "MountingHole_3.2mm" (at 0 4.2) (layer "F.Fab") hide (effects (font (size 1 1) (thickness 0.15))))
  (pad "" np_thru_hole circle locked (at 0 0) (size 3.2 3.2) (drill 3.2) (layers *.Cu *.Mask)))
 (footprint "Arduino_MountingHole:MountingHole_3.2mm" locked (layer "F.Cu") (at 190.17 49.2)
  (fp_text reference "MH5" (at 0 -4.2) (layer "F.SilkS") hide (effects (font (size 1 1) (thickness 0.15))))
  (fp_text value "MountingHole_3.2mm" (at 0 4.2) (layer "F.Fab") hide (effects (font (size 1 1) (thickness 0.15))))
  (pad "" np_thru_hole circle locked (at 0 0) (size 3.2 3.2) (drill 3.2) (layers *.Cu *.Mask)))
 (gr_line (start 196.5 37.5) (end 196.5 46.66) (layer "Edge.Cuts") (width 0.15))
 (gr_line (start 199.06 59.36) (end 201.6 61.9) (layer "Edge.Cuts") (width 0.15))
 (gr_line (start 100 99.238) (end 100 47.422) (layer "Edge.Cuts") (width 0.15))
 (gr_line (start 201.6 61.9) (end 201.6 96.19) (layer "Edge.Cuts") (width 0.15))
 (gr_line (start 198.298 100) (end 100.762 100) (layer "Edge.Cuts") (width 0.15))
 (gr_line (start 100.762 37.5) (end 196.5 37.5) (layer "Edge.Cuts") (width 0.15))
 (gr_arc (start 100.762 100) (mid 100.223185 99.776815) (end 100 99.238) (layer "Edge.Cuts") (width 0.15))
 (gr_line (start 201.6 96.19) (end 199.06 98.73) (layer "Edge.Cuts") (width 0.15))
 (gr_line (start 100.762 37.5) (end 100.762 46.66) (layer "Edge.Cuts") (width 0.15))
 (gr_line (start 196.5 46.66) (end 199.06 49.2) (layer "Edge.Cuts") (width 0.15))
 (gr_arc (start 199.06 99.238) (mid 198.836815 99.776815) (end 198.298 100) (layer "Edge.Cuts") (width 0.15))
 (gr_line (start 199.06 49.2) (end 199.06 59.36) (layer "Edge.Cuts") (width 0.15))
 (gr_line (start 199.06 98.73) (end 199.06 99.238) (layer "Edge.Cuts") (width 0.15))
 (gr_arc (start 100 47.422) (mid 100.223185 46.883185) (end 100.762 46.66) (layer "Edge.Cuts") (width 0.15))
 (segment (start 159.92 86.58) (end 160 86.5) (width 0.25) (layer "B.Cu") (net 1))
 (segment (start 143.5 47) (end 143 47) (width 0.25) (layer "B.Cu") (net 1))
 (segment (start 154.5 47) (end 154 47) (width 0.25) (layer "B.Cu") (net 1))
 (segment (start 146.2675 46.2675) (end 146.2675 43.1425) (width 0.25) (layer "B.Cu") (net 1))
 (segment (start 143.5 47) (end 126.5 47) (width 0.25) (layer "B.Cu") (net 1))
 (segment (start 150.5 47) (end 149.7675 46.2675) (width 0.25) (layer "B.Cu") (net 1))
 (segment (start 143 96) (end 143.18 96.18) (width 0.25) (layer "B.Cu") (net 1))
 (segment (start 178 47) (end 161 47) (width 0.25) (layer "B.Cu") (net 1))
 (segment (start 149.7675 46.2675) (end 149.7675 43.1425) (width 0.25) (layer "B.Cu") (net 1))
 (segment (start 143.18 96.18) (end 143.18 97.46) (width 0.25) (layer "B.Cu") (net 1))
 (segment (start 142.5 46.5) (end 142.5 43.41) (width 0.25) (layer "B.Cu") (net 1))
 (segment (start 154 47) (end 153.2675 46.2675) (width 0.25) (layer "B.Cu") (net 1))
 (segment (start 178.2675 46.7325) (end 178 47) (width 0.25) (layer "B.Cu") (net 1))
 (segment (start 144.42 86.58) (end 143 88) (width 0.25) (layer "B.Cu") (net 1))
 (segment (start 160.2675 46.2675) (end 160.2675 43.1425) (width 0.25) (layer "B.Cu") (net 1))
 (segment (start 147 47) (end 143.5 47) (width 0.25) (layer "B.Cu") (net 1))
 (segment (start 161 47) (end 160.2675 46.2675) (width 0.25) (layer "B.Cu") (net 1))
 (segment (start 153.2675 46.2675) (end 153.2675 43.1425) (width 0.25) (layer "B.Cu") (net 1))
 (segment (start 178.2675 43.1425) (end 178.2675 46.7325) (width 0.25) (layer "B.Cu") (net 1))
 (segment (start 154.5 47) (end 150.5 47) (width 0.25) (layer "B.Cu") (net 1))
 (segment (start 126.416 47.084) (end 126.416 49.2) (width 0.25) (layer "B.Cu") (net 1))
 (segment (start 142.5 43.41) (end 142.7675 43.1425) (width 0.25) (layer "B.Cu") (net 1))
 (segment (start 157.755 86.58) (end 187.755 86.58) (width 0.25) (layer "B.Cu") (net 1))
 (segment (start 126.5 47) (end 126.416 47.084) (width 0.25) (layer "B.Cu") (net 1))
 (segment (start 147 47) (end 146.2675 46.2675) (width 0.25) (layer "B.Cu") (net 1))
 (segment (start 161 47) (end 154.5 47) (width 0.25) (layer "B.Cu") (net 1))
 (segment (start 157.755 86.58) (end 144.42 86.58) (width 0.25) (layer "B.Cu") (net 1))
 (segment (start 143 88) (end 143 96) (width 0.25) (layer "B.Cu") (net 1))
 (segment (start 150.5 47) (end 147 47) (width 0.25) (layer "B.Cu") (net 1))
 (segment (start 143 47) (end 142.5 46.5) (width 0.25) (layer "B.Cu") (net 1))
 (segment (start 193.32 90.5) (end 193.98 89.84) (width 0.25) (layer "B.Cu") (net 2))
 (segment (start 161.5 90.5) (end 161.554 90.446) (width 0.25) (layer "B.Cu") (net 2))
 (segment (start 192.446 90.446) (end 192.5 90.5) (width 0.25) (layer "B.Cu") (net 2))
 (segment (start 192.7 87.3) (end 193.98 87.3) (width 0.25) (layer "B.Cu") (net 4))
 (segment (start 196.52 84.02) (end 196.52 84.76) (width 0.25) (layer "F.Cu") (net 7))
 (segment (start 169.46 84.04) (end 169.5 84) (width 0.25) (layer "B.Cu") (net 26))
 (segment (start 157.755 84.04) (end 169.46 84.04) (width 0.25) (layer "B.Cu") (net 26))
 (segment (start 169.5 84) (end 170.5 83) (width 0.25) (layer "B.Cu") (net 26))
 (segment (start 170.5 83) (end 170.5 59.5) (width 0.25) (layer "B.Cu") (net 26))
 (segment (start 170.5 59.5) (end 193 59.5) (width 0.25) (layer "B.Cu") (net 26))
 (segment (start 195.465 60.535) (end 195.5 60.5) (width 0.25) (layer "F.Cu") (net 27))
 (segment (start 186.465 60.535) (end 195.465 60.535) (width 0.25) (layer "F.Cu") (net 27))
 (segment (start 187.755 76.42) (end 185.92 76.42) (width 0.25) (layer "F.Cu") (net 27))
 (segment (start 185.5 76) (end 185.5 61.5) (width 0.25) (layer "F.Cu") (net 27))
 (segment (start 186 61) (end 186.465 60.535) (width 0.25) (layer "F.Cu") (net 27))
 (segment (start 195.5 60.5) (end 196 60) (width 0.25) (layer "F.Cu") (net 27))
 (segment (start 185.5 61.5) (end 186 61) (width 0.25) (layer "F.Cu") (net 27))
 (segment (start 185.92 76.42) (end 185.5 76) (width 0.25) (layer "F.Cu") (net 27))
 (segment (start 196 60) (end 196.5 60) (width 0.25) (layer "F.Cu") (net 27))
 (segment (start 169.5 57) (end 169.68 56.82) (width 0.25) (layer "B.Cu") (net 28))
 (segment (start 169 81.5) (end 169.5 81) (width 0.25) (layer "B.Cu") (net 28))
 (segment (start 157.755 81.5) (end 169 81.5) (width 0.25) (layer "B.Cu") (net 28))
 (segment (start 169.5 81) (end 169.5 57) (width 0.25) (layer "B.Cu") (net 28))
 (segment (start 169.68 56.82) (end 193.98 56.82) (width 0.25) (layer "B.Cu") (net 28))
 (segment (start 185 58) (end 195.5 58) (width 0.25) (layer "F.Cu") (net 29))
 (segment (start 195.5 58) (end 196 58) (width 0.25) (layer "F.Cu") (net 29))
 (segment (start 184.54 78.96) (end 184.5 79) (width 0.25) (layer "F.Cu") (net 29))
 (segment (start 196 58) (end 196.5 57.5) (width 0.25) (layer "F.Cu") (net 29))
 (segment (start 184.5 58.5) (end 185 58) (width 0.25) (layer "F.Cu") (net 29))
 (segment (start 184.5 79) (end 184.5 58.5) (width 0.25) (layer "F.Cu") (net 29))
 (segment (start 187.755 78.96) (end 184.54 78.96) (width 0.25) (layer "F.Cu") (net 29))
 (segment (start 163 78) (end 163 54.5) (width 0.25) (layer "B.Cu") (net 30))
 (segment (start 162.04 78.96) (end 163 78) (width 0.25) (layer "B.Cu") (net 30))
 (segment (start 163 54.5) (end 163.22 54.28) (width 0.25) (layer "B.Cu") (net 30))
 (segment (start 163.22 54.28) (end 193.98 54.28) (width 0.25) (layer "B.Cu") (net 30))
 (segment (start 157.755 78.96) (end 162.04 78.96) (width 0.25) (layer "B.Cu") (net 30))
 (segment (start 184 55.5) (end 195.5 55.5) (width 0.25) (layer "F.Cu") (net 31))
 (segment (start 196 55.5) (end 196.5 55) (width 0.25) (layer "F.Cu") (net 31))
 (segment (start 183.5 81) (end 183.5 56) (width 0.25) (layer "F.Cu") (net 31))
 (segment (start 195.5 55.5) (end 196 55.5) (width 0.25) (layer "F.Cu") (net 31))
 (segment (start 183.5 56) (end 184 55.5) (width 0.25) (layer "F.Cu") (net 31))
 (segment (start 184 81.5) (end 183.5 81) (width 0.25) (layer "F.Cu") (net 31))
 (segment (start 187.755 81.5) (end 184 81.5) (width 0.25) (layer "F.Cu") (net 31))
 (segment (start 160.5 52) (end 160.76 51.74) (width 0.25) (layer "B.Cu") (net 32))
 (segment (start 160.76 51.74) (end 193.98 51.74) (width 0.25) (layer "B.Cu") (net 32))
 (segment (start 160.08 76.42) (end 160.5 76) (width 0.25) (layer "B.Cu") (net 32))
 (segment (start 157.755 76.42) (end 160.08 76.42) (width 0.25) (layer "B.Cu") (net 32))
 (segment (start 160.5 76) (end 160.5 52) (width 0.25) (layer "B.Cu") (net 32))
 (segment (start 183 53) (end 195.5 53) (width 0.25) (layer "F.Cu") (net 33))
 (segment (start 183 84) (end 182.5 83.5) (width 0.25) (layer "F.Cu") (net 33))
 (segment (start 187.755 84.04) (end 183.04 84.04) (width 0.25) (layer "F.Cu") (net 33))
 (segment (start 182.5 53.5) (end 183 53) (width 0.25) (layer "F.Cu") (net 33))
 (segment (start 195.5 53) (end 196 53) (width 0.25) (layer "F.Cu") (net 33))
 (segment (start 182.5 83.5) (end 182.5 53.5) (width 0.25) (layer "F.Cu") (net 33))
 (segment (start 190 88.5) (end 190.165 88.665) (width 0.25) (layer "F.Cu") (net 33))
 (segment (start 183.04 84.04) (end 183 84) (width 0.25) (layer "F.Cu") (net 33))
 (segment (start 196 53) (end 196.5 52.5) (width 0.25) (layer "F.Cu") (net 33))
 (segment (start 157 40) (end 113 40) (width 0.25) (layer "B.Cu") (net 34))
 (segment (start 112 85) (end 114.5 87.5) (width 0.25) (layer "B.Cu") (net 34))
 (segment (start 157 40) (end 156.7675 40.2325) (width 0.25) (layer "B.Cu") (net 34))
 (segment (start 137.5 88) (end 137.5 97) (width 0.25) (layer "B.Cu") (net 34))
 (segment (start 174.7675 43.1425) (end 174.7675 40.2675) (width 0.25) (layer "B.Cu") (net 34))
 (segment (start 112 41) (end 112 85) (width 0.25) (layer "B.Cu") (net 34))
 (segment (start 137 87.5) (end 137.5 88) (width 0.25) (layer "B.Cu") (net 34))
 (segment (start 137.5 97) (end 137.96 97.46) (width 0.25) (layer "B.Cu") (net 34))
 (segment (start 174.7675 40.2675) (end 174.5 40) (width 0.25) (layer "B.Cu") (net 34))
 (segment (start 114.5 87.5) (end 137 87.5) (width 0.25) (layer "B.Cu") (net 34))
 (segment (start 156.7675 40.2325) (end 156.7675 43.1425) (width 0.25) (layer "B.Cu") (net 34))
 (segment (start 137.96 97.46) (end 138.1 97.46) (width 0.25) (layer "B.Cu") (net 34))
 (segment (start 113 40) (end 112 41) (width 0.25) (layer "B.Cu") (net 34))
 (segment (start 174.5 40) (end 157 40) (width 0.25) (layer "B.Cu") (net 34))
 (segment (start 157.755 93.755) (end 157.01 94.5) (width 0.25) (layer "F.Cu") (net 38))
 (segment (start 157.01 94.5) (end 136 94.5) (width 0.25) (layer "F.Cu") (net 38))
 (segment (start 187.755 94.245) (end 187.5 94.5) (width 0.25) (layer "F.Cu") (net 38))
 (segment (start 158.5 94.5) (end 157.755 93.755) (width 0.25) (layer "F.Cu") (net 38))
 (segment (start 157.755 93.755) (end 157.755 91.66) (width 0.25) (layer "F.Cu") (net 38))
 (segment (start 135.56 94.94) (end 135.56 97.46) (width 0.25) (layer "F.Cu") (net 38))
 (segment (start 187.5 94.5) (end 158.5 94.5) (width 0.25) (layer "F.Cu") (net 38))
 (segment (start 136 94.5) (end 135.56 94.94) (width 0.25) (layer "F.Cu") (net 38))
 (segment (start 187.755 91.66) (end 187.755 94.245) (width 0.25) (layer "F.Cu") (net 38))
 (segment (start 168.58 46.58) (end 167.7675 45.7675) (width 0.25) (layer "F.Cu") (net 73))
 (segment (start 167.7675 45.7675) (end 167.7675 43.1425) (width 0.25) (layer "F.Cu") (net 73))
 (segment (start 168.58 49.2) (end 168.58 46.58) (width 0.25) (layer "F.Cu") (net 73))
 (segment (start 171.12 49.2) (end 171.12 43.29) (width 0.25) (layer "F.Cu") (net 74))
 (segment (start 171.12 43.29) (end 171.2675 43.1425) (width 0.25) (layer "F.Cu") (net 74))
 (segment (start 175 46) (end 181.5 46) (width 0.25) (layer "F.Cu") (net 75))
 (segment (start 173.66 49.2) (end 173.66 47.34) (width 0.25) (layer "F.Cu") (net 75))
 (segment (start 181.7675 45.7325) (end 181.7675 43.1425) (width 0.25) (layer "F.Cu") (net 75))
 (segment (start 173.66 47.34) (end 175 46) (width 0.25) (layer "F.Cu") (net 75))
 (segment (start 181.5 46) (end 181.7675 45.7325) (width 0.25) (layer "F.Cu") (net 75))
 (segment (start 185.2675 46.2325) (end 185.2675 43.1425) (width 0.25) (layer "F.Cu") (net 76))
 (segment (start 176.5 47) (end 184.5 47) (width 0.25) (layer "F.Cu") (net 76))
 (segment (start 176.2 49.2) (end 176.2 47.3) (width 0.25) (layer "F.Cu") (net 76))
 (segment (start 184.5 47) (end 185.2675 46.2325) (width 0.25) (layer "F.Cu") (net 76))
 (segment (start 176.2 47.3) (end 176.5 47) (width 0.25) (layer "F.Cu") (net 76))
 (segment (start 105.6425 84.2325) (end 141.2675 84.2325) (width 0.25) (layer "F.Cu") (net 87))
 (segment (start 141.2675 84.2325) (end 141.5 84) (width 0.25) (layer "F.Cu") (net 87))
 (segment (start 141.5045 80.7325) (end 142.515 79.722) (width 0.25) (layer "F.Cu") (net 88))
 (segment (start 105.6425 80.7325) (end 141.5045 80.7325) (width 0.25) (layer "F.Cu") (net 88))
 (segment (start 134.7675 74.7325) (end 135 74.5) (width 0.25) (layer "F.Cu") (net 82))
 (segment (start 161.5 83) (end 161.778 83.278) (width 0.25) (layer "F.Cu") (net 82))
 (segment (start 161.5 68) (end 161.5 83) (width 0.25) (layer "F.Cu") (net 82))
 (segment (start 161.778 83.278) (end 172.515 83.278) (width 0.25) (layer "F.Cu") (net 82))
 (segment (start 135 74.5) (end 135 68) (width 0.25) (layer "F.Cu") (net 82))
 (segment (start 135 68) (end 161.5 68) (width 0.25) (layer "F.Cu") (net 82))
 (segment (start 105.6425 74.7325) (end 134.7675 74.7325) (width 0.25) (layer "F.Cu") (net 82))
 (segment (start 133.7675 71.2325) (end 134 71) (width 0.25) (layer "F.Cu") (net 83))
 (segment (start 168.5 67.5) (end 168.5 79.5) (width 0.25) (layer "F.Cu") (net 83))
 (segment (start 168 67) (end 168.5 67.5) (width 0.25) (layer "F.Cu") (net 83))
 (segment (start 134 67) (end 168 67) (width 0.25) (layer "F.Cu") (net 83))
 (segment (start 105.6425 71.2325) (end 133.7675 71.2325) (width 0.25) (layer "F.Cu") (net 83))
 (segment (start 168.722 79.722) (end 172.515 79.722) (width 0.25) (layer "F.Cu") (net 83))
 (segment (start 168.5 79.5) (end 168.722 79.722) (width 0.25) (layer "F.Cu") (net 83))
 (segment (start 134 71) (end 134 67) (width 0.25) (layer "F.Cu") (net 83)))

